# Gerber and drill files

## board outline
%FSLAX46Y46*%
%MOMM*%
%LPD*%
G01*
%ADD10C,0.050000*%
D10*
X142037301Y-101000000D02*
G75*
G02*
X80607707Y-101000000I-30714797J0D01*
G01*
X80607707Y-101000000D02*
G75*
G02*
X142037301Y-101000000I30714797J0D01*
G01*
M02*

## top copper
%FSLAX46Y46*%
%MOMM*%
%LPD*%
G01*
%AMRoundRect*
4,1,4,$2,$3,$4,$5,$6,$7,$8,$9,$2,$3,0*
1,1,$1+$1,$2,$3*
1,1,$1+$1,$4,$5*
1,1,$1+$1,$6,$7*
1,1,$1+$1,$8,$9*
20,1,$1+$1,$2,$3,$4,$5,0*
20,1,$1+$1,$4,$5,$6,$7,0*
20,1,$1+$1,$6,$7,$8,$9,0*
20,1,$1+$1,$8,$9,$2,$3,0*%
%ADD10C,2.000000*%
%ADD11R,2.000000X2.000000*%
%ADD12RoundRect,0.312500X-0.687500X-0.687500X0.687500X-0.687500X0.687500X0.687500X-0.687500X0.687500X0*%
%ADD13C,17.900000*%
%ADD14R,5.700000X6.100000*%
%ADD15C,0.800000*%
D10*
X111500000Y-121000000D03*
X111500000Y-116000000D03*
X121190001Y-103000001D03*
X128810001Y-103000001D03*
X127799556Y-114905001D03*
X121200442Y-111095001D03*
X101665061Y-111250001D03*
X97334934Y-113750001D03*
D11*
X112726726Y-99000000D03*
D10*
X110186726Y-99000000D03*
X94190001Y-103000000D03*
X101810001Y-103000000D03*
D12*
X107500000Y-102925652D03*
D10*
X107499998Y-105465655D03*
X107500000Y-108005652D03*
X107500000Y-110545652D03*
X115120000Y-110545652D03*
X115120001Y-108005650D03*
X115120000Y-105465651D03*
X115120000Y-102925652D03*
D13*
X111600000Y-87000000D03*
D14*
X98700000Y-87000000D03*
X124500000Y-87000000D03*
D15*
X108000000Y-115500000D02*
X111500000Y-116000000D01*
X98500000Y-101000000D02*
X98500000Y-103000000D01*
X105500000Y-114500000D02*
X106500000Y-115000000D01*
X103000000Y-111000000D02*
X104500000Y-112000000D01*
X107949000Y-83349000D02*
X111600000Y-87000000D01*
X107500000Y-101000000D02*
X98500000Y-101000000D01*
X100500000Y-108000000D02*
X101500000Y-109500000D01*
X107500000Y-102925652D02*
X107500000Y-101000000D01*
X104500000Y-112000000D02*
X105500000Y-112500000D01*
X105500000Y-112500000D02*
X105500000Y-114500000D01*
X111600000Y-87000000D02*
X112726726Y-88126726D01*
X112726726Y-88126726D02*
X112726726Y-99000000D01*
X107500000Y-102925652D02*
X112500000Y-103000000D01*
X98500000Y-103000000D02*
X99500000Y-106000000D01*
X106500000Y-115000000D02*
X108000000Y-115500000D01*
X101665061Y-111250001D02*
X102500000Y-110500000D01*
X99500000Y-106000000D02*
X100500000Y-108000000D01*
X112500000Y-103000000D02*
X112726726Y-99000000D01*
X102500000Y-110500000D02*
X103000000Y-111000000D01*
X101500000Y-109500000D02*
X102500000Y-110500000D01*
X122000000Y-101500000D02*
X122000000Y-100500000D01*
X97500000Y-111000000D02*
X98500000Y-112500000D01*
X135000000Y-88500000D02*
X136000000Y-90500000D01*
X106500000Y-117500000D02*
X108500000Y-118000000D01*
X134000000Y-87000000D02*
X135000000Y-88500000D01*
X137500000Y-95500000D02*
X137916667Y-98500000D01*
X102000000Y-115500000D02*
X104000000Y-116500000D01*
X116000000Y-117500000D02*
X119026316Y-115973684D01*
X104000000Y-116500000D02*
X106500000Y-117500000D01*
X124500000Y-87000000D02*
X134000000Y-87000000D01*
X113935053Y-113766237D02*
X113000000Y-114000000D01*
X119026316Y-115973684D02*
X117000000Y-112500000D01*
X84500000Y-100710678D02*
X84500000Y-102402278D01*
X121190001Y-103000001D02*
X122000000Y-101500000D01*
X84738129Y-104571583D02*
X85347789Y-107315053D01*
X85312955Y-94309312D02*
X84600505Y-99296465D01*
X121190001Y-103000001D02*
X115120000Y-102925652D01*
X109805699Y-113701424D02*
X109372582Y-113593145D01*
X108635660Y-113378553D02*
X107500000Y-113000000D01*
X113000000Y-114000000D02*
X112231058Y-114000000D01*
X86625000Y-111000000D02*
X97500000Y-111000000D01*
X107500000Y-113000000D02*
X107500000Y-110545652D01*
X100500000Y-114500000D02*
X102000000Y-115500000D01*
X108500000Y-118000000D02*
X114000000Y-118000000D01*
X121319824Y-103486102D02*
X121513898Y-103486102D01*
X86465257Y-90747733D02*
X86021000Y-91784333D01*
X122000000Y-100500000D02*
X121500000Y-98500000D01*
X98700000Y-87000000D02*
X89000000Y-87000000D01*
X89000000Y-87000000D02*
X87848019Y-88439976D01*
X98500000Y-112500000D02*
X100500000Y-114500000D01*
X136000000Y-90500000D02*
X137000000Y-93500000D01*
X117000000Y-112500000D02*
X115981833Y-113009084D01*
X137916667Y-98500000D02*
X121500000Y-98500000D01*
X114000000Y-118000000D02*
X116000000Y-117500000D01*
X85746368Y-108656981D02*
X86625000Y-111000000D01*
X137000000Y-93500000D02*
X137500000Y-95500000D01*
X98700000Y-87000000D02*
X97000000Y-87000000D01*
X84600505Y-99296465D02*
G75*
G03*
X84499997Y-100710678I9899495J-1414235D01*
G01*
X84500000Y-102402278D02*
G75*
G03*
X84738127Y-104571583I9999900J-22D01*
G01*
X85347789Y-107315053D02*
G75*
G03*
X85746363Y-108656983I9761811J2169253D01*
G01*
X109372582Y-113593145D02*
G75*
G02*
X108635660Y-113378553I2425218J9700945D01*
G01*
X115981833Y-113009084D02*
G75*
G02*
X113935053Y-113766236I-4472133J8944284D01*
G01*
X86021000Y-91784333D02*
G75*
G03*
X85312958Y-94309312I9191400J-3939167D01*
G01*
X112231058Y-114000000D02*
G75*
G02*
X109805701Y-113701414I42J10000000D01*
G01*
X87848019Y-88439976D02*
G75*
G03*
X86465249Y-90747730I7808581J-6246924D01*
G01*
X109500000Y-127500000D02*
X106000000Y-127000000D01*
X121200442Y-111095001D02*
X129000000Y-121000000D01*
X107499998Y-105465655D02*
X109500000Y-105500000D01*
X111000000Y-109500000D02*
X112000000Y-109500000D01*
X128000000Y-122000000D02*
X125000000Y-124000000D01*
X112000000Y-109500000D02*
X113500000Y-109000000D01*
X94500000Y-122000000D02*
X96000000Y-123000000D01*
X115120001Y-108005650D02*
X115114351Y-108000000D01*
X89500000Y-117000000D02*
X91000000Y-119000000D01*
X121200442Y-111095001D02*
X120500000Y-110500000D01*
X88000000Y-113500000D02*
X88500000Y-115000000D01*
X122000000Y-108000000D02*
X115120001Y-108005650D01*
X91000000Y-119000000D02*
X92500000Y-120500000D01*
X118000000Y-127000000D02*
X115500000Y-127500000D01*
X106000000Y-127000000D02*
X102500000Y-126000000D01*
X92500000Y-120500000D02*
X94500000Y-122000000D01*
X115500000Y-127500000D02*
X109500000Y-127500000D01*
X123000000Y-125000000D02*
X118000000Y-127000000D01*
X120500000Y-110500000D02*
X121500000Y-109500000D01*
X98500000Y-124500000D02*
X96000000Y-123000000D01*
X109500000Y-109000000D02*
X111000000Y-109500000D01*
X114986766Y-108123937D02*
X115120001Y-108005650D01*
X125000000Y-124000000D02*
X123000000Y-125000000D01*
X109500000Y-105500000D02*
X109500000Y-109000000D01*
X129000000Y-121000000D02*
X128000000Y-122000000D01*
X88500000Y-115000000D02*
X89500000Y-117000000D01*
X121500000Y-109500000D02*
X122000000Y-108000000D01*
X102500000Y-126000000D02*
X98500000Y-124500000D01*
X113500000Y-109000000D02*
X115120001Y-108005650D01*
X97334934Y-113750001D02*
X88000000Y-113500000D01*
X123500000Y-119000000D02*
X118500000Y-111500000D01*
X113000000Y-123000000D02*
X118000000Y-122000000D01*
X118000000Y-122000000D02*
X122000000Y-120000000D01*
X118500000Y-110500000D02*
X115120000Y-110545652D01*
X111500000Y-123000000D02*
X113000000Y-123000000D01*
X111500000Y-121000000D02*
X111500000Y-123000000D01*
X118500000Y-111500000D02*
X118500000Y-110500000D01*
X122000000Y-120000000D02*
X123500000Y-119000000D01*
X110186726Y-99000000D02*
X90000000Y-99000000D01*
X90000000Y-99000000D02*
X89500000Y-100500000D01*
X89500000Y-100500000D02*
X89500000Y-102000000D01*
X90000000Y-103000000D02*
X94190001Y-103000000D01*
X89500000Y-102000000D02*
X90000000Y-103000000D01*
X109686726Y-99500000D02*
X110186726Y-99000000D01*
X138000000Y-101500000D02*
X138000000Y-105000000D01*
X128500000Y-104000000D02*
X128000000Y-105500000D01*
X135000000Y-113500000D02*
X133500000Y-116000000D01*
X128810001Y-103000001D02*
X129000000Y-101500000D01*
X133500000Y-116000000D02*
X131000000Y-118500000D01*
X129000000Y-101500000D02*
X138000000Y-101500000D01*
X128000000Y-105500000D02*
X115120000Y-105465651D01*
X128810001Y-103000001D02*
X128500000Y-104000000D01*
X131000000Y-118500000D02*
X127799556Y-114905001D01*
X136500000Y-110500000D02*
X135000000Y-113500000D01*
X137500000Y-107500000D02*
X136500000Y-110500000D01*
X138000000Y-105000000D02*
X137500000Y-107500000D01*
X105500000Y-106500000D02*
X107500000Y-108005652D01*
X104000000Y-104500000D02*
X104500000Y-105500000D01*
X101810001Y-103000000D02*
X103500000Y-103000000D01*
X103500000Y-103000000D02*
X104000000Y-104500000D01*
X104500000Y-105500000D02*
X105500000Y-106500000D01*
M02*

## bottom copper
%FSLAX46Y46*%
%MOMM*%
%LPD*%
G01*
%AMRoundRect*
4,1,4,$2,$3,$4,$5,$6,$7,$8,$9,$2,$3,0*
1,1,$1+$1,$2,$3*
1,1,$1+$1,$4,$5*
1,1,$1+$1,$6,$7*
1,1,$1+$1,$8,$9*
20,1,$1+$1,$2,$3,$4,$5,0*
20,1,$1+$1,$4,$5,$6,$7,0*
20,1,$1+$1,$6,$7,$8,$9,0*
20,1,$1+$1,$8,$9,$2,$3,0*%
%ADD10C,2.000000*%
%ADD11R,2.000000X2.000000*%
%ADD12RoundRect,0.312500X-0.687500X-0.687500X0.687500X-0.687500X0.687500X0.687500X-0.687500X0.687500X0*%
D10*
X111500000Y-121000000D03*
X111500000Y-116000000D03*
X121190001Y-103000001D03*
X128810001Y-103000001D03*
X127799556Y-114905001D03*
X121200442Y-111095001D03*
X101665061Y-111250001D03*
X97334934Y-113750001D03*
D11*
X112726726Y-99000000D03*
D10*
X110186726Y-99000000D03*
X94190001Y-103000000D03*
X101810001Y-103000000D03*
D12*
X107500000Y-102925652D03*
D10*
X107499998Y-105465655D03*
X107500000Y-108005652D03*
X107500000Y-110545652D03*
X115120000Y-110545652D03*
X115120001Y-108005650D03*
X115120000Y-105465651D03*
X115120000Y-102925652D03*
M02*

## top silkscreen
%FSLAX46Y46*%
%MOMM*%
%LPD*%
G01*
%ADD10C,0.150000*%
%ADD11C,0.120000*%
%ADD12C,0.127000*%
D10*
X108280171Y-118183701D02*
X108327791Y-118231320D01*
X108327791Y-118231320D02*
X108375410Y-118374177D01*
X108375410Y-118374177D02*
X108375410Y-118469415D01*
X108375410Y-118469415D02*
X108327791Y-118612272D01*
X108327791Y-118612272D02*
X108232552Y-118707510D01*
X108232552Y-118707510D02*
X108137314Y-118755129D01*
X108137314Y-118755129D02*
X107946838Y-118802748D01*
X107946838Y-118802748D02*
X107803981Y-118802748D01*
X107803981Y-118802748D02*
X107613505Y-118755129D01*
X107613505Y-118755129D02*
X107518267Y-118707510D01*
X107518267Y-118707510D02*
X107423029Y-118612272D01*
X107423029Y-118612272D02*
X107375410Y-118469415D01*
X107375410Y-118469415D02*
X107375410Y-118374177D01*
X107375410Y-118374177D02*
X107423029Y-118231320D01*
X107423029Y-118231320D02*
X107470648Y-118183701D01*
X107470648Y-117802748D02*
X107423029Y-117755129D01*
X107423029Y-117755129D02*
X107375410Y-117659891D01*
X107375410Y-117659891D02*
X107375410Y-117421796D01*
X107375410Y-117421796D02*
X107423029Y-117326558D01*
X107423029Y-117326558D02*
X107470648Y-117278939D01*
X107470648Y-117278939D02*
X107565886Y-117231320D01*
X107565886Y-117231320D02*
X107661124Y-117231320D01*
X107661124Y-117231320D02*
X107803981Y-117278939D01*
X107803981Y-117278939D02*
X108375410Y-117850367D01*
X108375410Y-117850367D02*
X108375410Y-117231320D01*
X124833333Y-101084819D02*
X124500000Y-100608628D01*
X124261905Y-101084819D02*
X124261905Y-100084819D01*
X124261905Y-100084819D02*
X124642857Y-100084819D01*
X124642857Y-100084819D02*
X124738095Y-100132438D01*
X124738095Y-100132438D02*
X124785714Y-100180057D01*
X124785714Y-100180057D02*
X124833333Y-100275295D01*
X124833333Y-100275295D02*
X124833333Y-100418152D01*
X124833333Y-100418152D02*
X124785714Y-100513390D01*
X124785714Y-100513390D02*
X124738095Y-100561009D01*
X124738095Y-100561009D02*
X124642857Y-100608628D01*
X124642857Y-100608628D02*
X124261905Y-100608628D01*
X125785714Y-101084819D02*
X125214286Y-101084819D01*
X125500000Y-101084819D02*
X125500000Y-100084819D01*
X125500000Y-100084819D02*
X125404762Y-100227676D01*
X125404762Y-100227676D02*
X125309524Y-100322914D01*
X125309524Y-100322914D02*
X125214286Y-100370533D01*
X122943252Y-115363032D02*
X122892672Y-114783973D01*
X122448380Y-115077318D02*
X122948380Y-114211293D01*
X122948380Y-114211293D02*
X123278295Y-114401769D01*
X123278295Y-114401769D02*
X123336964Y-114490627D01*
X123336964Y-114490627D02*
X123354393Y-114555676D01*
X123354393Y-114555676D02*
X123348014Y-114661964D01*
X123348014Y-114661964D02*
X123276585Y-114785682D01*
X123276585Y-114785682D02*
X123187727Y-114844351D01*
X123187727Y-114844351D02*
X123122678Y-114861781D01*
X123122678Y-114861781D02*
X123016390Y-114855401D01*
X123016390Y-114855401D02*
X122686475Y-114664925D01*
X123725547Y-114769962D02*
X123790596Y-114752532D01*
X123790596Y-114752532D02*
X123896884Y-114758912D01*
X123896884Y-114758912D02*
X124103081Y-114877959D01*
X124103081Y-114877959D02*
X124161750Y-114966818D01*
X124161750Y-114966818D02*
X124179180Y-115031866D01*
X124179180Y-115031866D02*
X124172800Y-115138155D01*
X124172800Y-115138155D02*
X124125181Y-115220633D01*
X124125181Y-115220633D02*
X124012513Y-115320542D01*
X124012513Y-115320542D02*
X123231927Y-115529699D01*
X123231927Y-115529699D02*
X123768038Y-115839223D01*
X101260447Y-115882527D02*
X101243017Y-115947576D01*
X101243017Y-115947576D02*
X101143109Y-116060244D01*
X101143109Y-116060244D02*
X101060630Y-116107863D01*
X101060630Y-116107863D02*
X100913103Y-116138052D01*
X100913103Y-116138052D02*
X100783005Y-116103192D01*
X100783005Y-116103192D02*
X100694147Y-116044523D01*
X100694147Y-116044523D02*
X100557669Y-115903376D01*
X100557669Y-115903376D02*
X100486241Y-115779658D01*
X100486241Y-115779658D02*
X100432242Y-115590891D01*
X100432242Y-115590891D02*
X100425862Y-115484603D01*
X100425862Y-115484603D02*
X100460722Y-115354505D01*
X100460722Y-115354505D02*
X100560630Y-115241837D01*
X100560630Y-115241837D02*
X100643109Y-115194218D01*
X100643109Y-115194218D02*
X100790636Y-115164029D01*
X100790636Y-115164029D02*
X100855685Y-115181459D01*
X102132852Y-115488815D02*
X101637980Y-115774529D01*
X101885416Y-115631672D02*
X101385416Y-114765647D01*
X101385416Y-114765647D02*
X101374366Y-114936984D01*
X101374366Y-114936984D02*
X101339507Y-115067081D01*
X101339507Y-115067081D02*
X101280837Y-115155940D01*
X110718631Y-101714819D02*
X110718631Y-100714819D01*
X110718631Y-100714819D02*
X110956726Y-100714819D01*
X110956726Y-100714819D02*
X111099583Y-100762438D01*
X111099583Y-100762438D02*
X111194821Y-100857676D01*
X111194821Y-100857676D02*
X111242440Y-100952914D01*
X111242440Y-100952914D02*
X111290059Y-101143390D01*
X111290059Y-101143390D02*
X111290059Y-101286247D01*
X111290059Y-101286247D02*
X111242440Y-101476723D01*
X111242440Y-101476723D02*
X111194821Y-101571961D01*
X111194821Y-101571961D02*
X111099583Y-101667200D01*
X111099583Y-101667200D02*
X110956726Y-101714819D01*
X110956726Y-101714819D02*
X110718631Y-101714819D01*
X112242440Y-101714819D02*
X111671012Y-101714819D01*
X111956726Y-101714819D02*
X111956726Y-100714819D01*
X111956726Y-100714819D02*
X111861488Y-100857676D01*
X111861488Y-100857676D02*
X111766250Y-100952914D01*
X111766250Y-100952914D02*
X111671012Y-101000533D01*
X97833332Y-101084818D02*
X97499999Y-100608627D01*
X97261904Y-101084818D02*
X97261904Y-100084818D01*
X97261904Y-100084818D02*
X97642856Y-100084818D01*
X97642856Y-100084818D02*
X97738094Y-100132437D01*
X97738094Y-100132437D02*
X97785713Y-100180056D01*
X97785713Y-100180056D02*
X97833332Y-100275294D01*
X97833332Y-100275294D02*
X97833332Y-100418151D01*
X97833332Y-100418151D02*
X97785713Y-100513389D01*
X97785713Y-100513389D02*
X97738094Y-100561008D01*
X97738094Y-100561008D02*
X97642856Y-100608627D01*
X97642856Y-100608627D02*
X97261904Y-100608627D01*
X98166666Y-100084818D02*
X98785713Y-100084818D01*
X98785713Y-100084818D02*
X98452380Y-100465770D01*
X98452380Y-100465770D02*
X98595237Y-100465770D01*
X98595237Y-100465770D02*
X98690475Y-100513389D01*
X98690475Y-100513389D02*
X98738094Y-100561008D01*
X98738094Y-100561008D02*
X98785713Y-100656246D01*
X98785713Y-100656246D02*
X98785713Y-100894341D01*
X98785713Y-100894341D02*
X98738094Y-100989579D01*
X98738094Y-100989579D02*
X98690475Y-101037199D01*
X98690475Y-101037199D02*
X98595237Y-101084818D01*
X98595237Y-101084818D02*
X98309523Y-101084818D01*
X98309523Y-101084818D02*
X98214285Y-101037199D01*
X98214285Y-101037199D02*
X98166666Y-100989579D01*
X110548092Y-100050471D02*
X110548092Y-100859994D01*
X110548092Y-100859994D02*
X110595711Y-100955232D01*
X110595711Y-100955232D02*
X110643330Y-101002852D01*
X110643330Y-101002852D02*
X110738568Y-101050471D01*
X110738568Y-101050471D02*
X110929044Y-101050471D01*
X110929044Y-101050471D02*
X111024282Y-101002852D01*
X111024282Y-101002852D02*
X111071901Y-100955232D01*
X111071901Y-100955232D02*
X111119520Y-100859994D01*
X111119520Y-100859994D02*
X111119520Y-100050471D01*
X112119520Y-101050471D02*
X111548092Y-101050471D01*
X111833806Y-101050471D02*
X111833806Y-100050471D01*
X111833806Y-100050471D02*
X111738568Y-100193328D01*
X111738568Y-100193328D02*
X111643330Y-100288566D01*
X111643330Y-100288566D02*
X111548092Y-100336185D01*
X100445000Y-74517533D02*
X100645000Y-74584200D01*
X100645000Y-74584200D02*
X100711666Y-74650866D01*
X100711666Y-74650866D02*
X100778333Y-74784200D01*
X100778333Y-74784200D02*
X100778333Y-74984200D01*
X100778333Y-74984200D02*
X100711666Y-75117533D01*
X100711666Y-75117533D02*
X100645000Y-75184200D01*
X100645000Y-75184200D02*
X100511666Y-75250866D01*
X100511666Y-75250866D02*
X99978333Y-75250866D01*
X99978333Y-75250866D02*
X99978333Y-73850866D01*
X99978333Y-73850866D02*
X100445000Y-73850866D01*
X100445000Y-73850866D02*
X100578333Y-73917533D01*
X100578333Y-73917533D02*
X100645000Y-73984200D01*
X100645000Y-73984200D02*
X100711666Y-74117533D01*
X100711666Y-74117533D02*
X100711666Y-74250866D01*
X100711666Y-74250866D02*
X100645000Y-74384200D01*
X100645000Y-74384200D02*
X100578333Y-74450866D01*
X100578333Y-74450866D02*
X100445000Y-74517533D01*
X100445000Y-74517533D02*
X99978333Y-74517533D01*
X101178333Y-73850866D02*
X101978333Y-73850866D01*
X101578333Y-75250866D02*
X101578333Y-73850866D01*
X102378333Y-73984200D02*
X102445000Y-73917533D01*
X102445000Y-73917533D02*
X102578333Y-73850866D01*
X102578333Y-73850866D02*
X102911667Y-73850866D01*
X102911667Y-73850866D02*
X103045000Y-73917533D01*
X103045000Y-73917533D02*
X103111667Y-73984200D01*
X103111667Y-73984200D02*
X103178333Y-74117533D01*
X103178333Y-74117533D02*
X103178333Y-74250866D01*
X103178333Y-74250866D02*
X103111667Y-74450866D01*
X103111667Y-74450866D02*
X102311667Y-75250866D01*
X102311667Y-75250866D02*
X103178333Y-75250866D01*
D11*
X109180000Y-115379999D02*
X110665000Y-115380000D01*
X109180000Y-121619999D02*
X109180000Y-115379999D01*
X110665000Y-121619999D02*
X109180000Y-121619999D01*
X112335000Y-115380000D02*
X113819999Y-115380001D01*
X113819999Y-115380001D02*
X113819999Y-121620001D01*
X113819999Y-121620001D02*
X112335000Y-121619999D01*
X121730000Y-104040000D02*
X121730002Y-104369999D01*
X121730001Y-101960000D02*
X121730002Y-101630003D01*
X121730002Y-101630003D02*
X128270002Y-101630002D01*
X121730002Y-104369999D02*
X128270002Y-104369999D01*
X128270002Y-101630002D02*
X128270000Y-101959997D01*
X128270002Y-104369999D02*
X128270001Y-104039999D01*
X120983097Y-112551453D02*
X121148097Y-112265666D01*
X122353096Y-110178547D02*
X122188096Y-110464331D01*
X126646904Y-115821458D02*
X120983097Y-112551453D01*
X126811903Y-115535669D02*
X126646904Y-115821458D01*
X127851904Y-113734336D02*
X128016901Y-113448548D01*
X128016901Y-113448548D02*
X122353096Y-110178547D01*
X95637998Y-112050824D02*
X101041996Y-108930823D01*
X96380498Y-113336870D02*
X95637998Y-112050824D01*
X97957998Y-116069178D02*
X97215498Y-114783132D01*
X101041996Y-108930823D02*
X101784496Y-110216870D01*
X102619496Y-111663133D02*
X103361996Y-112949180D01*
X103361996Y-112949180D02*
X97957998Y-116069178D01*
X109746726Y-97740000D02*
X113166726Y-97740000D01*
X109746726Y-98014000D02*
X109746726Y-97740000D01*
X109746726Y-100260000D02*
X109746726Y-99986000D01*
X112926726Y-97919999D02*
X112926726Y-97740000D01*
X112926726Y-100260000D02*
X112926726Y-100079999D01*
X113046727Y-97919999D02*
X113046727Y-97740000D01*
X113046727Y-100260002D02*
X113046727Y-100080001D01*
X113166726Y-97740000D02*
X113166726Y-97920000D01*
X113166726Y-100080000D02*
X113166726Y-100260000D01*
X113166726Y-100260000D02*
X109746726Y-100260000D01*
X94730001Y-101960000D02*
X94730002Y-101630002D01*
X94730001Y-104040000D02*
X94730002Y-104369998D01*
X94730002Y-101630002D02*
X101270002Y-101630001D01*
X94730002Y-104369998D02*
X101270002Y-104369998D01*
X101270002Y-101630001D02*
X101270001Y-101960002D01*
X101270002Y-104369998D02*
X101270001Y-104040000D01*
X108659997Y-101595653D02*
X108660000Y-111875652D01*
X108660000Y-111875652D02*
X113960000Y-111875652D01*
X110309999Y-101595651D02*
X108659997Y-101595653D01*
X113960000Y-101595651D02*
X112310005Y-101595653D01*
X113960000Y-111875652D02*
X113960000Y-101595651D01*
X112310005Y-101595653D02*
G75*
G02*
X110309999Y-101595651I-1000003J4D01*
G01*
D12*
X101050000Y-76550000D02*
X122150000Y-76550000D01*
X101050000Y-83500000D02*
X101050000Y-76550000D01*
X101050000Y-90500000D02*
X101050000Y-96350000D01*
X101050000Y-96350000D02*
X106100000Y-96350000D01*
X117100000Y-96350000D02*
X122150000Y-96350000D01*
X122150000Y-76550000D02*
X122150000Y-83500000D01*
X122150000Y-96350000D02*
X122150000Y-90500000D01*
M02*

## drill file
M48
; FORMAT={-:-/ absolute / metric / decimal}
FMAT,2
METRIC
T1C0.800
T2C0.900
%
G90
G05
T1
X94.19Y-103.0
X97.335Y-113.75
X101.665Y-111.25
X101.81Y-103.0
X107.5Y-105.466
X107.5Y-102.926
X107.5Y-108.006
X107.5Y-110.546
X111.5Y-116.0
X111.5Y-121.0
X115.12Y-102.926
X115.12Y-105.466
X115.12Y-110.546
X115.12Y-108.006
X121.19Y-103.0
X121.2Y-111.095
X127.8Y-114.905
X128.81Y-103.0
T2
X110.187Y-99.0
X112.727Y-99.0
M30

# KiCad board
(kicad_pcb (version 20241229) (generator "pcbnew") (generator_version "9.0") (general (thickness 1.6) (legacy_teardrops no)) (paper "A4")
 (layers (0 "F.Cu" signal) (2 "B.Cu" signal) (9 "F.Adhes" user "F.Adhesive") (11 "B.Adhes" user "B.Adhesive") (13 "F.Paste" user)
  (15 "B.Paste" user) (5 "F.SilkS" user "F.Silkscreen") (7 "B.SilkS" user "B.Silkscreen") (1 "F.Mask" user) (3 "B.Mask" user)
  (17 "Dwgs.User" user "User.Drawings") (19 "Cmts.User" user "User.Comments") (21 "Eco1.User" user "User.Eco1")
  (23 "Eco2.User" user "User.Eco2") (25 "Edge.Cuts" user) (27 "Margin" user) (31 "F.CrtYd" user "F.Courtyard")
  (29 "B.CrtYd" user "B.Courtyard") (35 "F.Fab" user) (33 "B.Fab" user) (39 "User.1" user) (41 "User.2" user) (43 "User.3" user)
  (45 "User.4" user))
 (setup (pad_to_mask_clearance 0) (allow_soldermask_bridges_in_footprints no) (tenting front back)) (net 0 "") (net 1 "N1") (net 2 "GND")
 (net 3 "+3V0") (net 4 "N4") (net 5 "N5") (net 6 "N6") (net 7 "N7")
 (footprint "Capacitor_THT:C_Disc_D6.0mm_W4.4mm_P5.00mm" (layer "F.Cu") (at 111.5 121 90)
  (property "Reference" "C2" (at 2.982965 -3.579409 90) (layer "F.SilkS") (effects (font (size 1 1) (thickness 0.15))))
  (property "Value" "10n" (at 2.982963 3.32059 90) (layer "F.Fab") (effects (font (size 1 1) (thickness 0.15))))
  (fp_line (start 5.620001 -2.32) (end 5.62 -0.835) (stroke (width 0.12) (type solid)) (layer "F.SilkS"))
  (fp_line (start -0.619999 -2.32) (end 5.620001 -2.32) (stroke (width 0.12) (type solid)) (layer "F.SilkS"))
  (fp_line (start -0.619999 -0.835) (end -0.619999 -2.32) (stroke (width 0.12) (type solid)) (layer "F.SilkS"))
  (fp_line (start 5.62 0.835) (end 5.619999 2.319999) (stroke (width 0.12) (type solid)) (layer "F.SilkS"))
  (fp_line (start 5.619999 2.319999) (end -0.620001 2.319999) (stroke (width 0.12) (type solid)) (layer "F.SilkS"))
  (fp_line (start -0.620001 2.319999) (end -0.619999 0.835) (stroke (width 0.12) (type solid)) (layer "F.SilkS"))
  (pad "1" thru_hole circle (at 0 0 90) (size 2 2) (drill 0.8) (layers "*.Cu" "*.Mask") (remove_unused_layers no) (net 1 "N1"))
  (pad "2" thru_hole circle (at 5 0 90) (size 2 2) (drill 0.8) (layers "*.Cu" "*.Mask") (remove_unused_layers no) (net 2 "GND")))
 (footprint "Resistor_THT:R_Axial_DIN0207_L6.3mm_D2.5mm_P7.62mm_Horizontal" (layer "F.Cu") (at 121.190001 103.000001)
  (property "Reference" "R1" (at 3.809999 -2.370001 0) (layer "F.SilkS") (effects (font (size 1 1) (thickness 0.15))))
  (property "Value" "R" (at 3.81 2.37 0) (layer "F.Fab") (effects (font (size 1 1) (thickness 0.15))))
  (fp_line (start 0.539999 1.039999) (end 0.540001 1.369998) (stroke (width 0.12) (type solid)) (layer "F.SilkS"))
  (fp_line (start 0.54 -1.040001) (end 0.540001 -1.369998) (stroke (width 0.12) (type solid)) (layer "F.SilkS"))
  (fp_line (start 0.540001 -1.369998) (end 7.080001 -1.369999) (stroke (width 0.12) (type solid)) (layer "F.SilkS"))
  (fp_line (start 0.540001 1.369998) (end 7.080001 1.369998) (stroke (width 0.12) (type solid)) (layer "F.SilkS"))
  (fp_line (start 7.080001 -1.369999) (end 7.079999 -1.040004) (stroke (width 0.12) (type solid)) (layer "F.SilkS"))
  (fp_line (start 7.080001 1.369998) (end 7.08 1.039998) (stroke (width 0.12) (type solid)) (layer "F.SilkS"))
  (pad "1" thru_hole circle (at 0 0) (size 2 2) (drill 0.8) (layers "*.Cu" "*.Mask") (remove_unused_layers no) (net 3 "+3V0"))
  (pad "2" thru_hole circle (at 7.62 0) (size 2 2) (drill 0.8) (layers "*.Cu" "*.Mask") (remove_unused_layers no) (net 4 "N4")))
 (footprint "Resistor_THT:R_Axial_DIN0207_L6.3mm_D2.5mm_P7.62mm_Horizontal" (layer "F.Cu") (at 127.799556 114.905001 150)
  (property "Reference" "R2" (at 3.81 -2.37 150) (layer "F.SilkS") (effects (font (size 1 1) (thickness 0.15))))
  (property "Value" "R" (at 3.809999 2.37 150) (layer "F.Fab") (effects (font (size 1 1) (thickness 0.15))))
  (fp_line (start 7.080001 -1.369997) (end 7.08 -1.039998) (stroke (width 0.12) (type solid)) (layer "F.SilkS"))
  (fp_line (start 7.08 1.369999) (end 7.080002 1.040003) (stroke (width 0.12) (type solid)) (layer "F.SilkS"))
  (fp_line (start 0.539997 -1.370001) (end 7.080001 -1.369997) (stroke (width 0.12) (type solid)) (layer "F.SilkS"))
  (fp_line (start 0.539999 -1.040001) (end 0.539997 -1.370001) (stroke (width 0.12) (type solid)) (layer "F.SilkS"))
  (fp_line (start 0.539998 1.04) (end 0.54 1.369998) (stroke (width 0.12) (type solid)) (layer "F.SilkS"))
  (fp_line (start 0.54 1.369998) (end 7.08 1.369999) (stroke (width 0.12) (type solid)) (layer "F.SilkS"))
  (pad "1" thru_hole circle (at 0 0 150) (size 2 2) (drill 0.8) (layers "*.Cu" "*.Mask") (remove_unused_layers no) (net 4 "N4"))
  (pad "2" thru_hole circle (at 7.62 0 150) (size 2 2) (drill 0.8) (layers "*.Cu" "*.Mask") (remove_unused_layers no) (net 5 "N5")))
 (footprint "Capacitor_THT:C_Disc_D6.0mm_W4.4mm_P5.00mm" (layer "F.Cu") (at 101.665061 111.250001 -150)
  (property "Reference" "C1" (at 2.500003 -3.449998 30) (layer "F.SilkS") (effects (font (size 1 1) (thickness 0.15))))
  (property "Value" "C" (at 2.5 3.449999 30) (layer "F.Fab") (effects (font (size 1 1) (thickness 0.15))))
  (fp_line (start 5.620001 2.319998) (end -0.619999 2.32) (stroke (width 0.12) (type solid)) (layer "F.SilkS"))
  (fp_line (start 5.62 0.835) (end 5.620001 2.319998) (stroke (width 0.12) (type solid)) (layer "F.SilkS"))
  (fp_line (start 5.619999 -2.319998) (end 5.62 -0.835) (stroke (width 0.12) (type solid)) (layer "F.SilkS"))
  (fp_line (start -0.619999 2.32) (end -0.619999 0.835) (stroke (width 0.12) (type solid)) (layer "F.SilkS"))
  (fp_line (start -0.619999 -0.835) (end -0.619999 -2.32) (stroke (width 0.12) (type solid)) (layer "F.SilkS"))
  (fp_line (start -0.619999 -2.32) (end 5.619999 -2.319998) (stroke (width 0.12) (type solid)) (layer "F.SilkS"))
  (pad "1" thru_hole circle (at 0 0 210) (size 2 2) (drill 0.8) (layers "*.Cu" "*.Mask") (remove_unused_layers no) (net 2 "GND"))
  (pad "2" thru_hole circle (at 5 0 210) (size 2 2) (drill 0.8) (layers "*.Cu" "*.Mask") (remove_unused_layers no) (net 5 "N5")))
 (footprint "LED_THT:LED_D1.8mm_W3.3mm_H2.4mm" (layer "F.Cu") (at 112.726726 99 180)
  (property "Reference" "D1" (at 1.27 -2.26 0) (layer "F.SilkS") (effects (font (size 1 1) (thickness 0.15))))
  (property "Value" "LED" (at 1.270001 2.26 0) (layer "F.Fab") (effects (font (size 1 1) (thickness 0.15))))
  (fp_line (start 2.98 1.26) (end -0.44 1.26) (stroke (width 0.12) (type solid)) (layer "F.SilkS"))
  (fp_line (start 2.98 0.986) (end 2.98 1.26) (stroke (width 0.12) (type solid)) (layer "F.SilkS"))
  (fp_line (start 2.98 -1.26) (end 2.98 -0.986) (stroke (width 0.12) (type solid)) (layer "F.SilkS"))
  (fp_line (start -0.2 1.080001) (end -0.2 1.26) (stroke (width 0.12) (type solid)) (layer "F.SilkS"))
  (fp_line (start -0.2 -1.26) (end -0.2 -1.079999) (stroke (width 0.12) (type solid)) (layer "F.SilkS"))
  (fp_line (start -0.320001 1.080001) (end -0.320001 1.26) (stroke (width 0.12) (type solid)) (layer "F.SilkS"))
  (fp_line (start -0.320001 -1.260002) (end -0.320001 -1.080001) (stroke (width 0.12) (type solid)) (layer "F.SilkS"))
  (fp_line (start -0.44 1.26) (end -0.44 1.08) (stroke (width 0.12) (type solid)) (layer "F.SilkS"))
  (fp_line (start -0.44 -1.08) (end -0.44 -1.26) (stroke (width 0.12) (type solid)) (layer "F.SilkS"))
  (fp_line (start -0.44 -1.26) (end 2.98 -1.26) (stroke (width 0.12) (type solid)) (layer "F.SilkS"))
  (pad "1" thru_hole rect (at 0 0 180) (size 2 2) (drill 0.9) (layers "*.Cu" "*.Mask") (remove_unused_layers no) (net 2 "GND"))
  (pad "2" thru_hole circle (at 2.54 0 180) (size 2 2) (drill 0.9) (layers "*.Cu" "*.Mask") (remove_unused_layers no) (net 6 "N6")))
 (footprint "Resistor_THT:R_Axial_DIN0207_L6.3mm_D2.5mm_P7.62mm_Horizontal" (layer "F.Cu") (at 94.190001 103)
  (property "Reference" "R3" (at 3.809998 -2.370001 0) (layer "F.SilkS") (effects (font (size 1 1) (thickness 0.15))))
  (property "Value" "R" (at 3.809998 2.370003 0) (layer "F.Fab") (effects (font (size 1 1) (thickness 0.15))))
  (fp_line (start 0.54 -1.04) (end 0.540001 -1.369998) (stroke (width 0.12) (type solid)) (layer "F.SilkS"))
  (fp_line (start 0.54 1.04) (end 0.540001 1.369998) (stroke (width 0.12) (type solid)) (layer "F.SilkS"))
  (fp_line (start 0.540001 -1.369998) (end 7.080001 -1.369999) (stroke (width 0.12) (type solid)) (layer "F.SilkS"))
  (fp_line (start 0.540001 1.369998) (end 7.080001 1.369998) (stroke (width 0.12) (type solid)) (layer "F.SilkS"))
  (fp_line (start 7.080001 -1.369999) (end 7.08 -1.039998) (stroke (width 0.12) (type solid)) (layer "F.SilkS"))
  (fp_line (start 7.080001 1.369998) (end 7.08 1.04) (stroke (width 0.12) (type solid)) (layer "F.SilkS"))
  (pad "1" thru_hole circle (at 0 0) (size 2 2) (drill 0.8) (layers "*.Cu" "*.Mask") (remove_unused_layers no) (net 6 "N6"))
  (pad "2" thru_hole circle (at 7.62 0) (size 2 2) (drill 0.8) (layers "*.Cu" "*.Mask") (remove_unused_layers no) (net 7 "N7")))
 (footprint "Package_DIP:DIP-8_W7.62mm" (layer "F.Cu") (at 107.5 102.925652)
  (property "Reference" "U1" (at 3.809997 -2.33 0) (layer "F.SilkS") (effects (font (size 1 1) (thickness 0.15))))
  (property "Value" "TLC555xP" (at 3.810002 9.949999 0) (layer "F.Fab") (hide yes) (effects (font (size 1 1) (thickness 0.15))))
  (fp_line (start 1.159997 -1.329999) (end 1.16 8.95) (stroke (width 0.12) (type solid)) (layer "F.SilkS"))
  (fp_line (start 1.16 8.95) (end 6.46 8.95) (stroke (width 0.12) (type solid)) (layer "F.SilkS"))
  (fp_line (start 2.809999 -1.330001) (end 1.159997 -1.329999) (stroke (width 0.12) (type solid)) (layer "F.SilkS"))
  (fp_line (start 6.46 -1.330001) (end 4.810005 -1.329999) (stroke (width 0.12) (type solid)) (layer "F.SilkS"))
  (fp_line (start 6.46 8.95) (end 6.46 -1.330001) (stroke (width 0.12) (type solid)) (layer "F.SilkS"))
  (fp_arc (start 4.810005 -1.329999) (mid 3.81 -0.33) (end 2.809999 -1.330001) (stroke (width 0.12) (type solid)) (layer "F.SilkS"))
  (pad "1" thru_hole roundrect (at 0 0) (size 2 2) (drill 0.8) (layers "*.Cu" "*.Mask") (remove_unused_layers no) (roundrect_rratio 0.15625)
   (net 2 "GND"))
  (pad "2" thru_hole circle (at -0.000002 2.540003) (size 2 2) (drill 0.8) (layers "*.Cu" "*.Mask") (remove_unused_layers no) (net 5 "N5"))
  (pad "3" thru_hole circle (at 0 5.08) (size 2 2) (drill 0.8) (layers "*.Cu" "*.Mask") (remove_unused_layers no) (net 7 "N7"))
  (pad "4" thru_hole circle (at 0 7.62) (size 2 2) (drill 0.8) (layers "*.Cu" "*.Mask") (remove_unused_layers no) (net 3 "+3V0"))
  (pad "5" thru_hole circle (at 7.62 7.62) (size 2 2) (drill 0.8) (layers "*.Cu" "*.Mask") (remove_unused_layers no) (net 1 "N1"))
  (pad "6" thru_hole circle (at 7.620001 5.079998) (size 2 2) (drill 0.8) (layers "*.Cu" "*.Mask") (remove_unused_layers no) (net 5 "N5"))
  (pad "7" thru_hole circle (at 7.62 2.539999) (size 2 2) (drill 0.8) (layers "*.Cu" "*.Mask") (remove_unused_layers no) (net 4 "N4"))
  (pad "8" thru_hole circle (at 7.62 0) (size 2 2) (drill 0.8) (layers "*.Cu" "*.Mask") (remove_unused_layers no) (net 3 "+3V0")))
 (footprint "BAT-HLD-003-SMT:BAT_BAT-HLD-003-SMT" (layer "F.Cu") (at 111.6 87)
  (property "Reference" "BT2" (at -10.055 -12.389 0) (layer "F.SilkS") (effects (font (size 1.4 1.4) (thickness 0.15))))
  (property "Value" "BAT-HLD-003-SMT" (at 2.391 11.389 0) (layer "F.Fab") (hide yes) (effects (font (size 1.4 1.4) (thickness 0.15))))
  (fp_line (start -10.55 -10.45) (end 10.55 -10.45) (stroke (width 0.127) (type solid)) (layer "F.SilkS"))
  (fp_line (start -10.55 -3.5) (end -10.55 -10.45) (stroke (width 0.127) (type solid)) (layer "F.SilkS"))
  (fp_line (start -10.55 3.5) (end -10.55 9.35) (stroke (width 0.127) (type solid)) (layer "F.SilkS"))
  (fp_line (start -10.55 9.35) (end -5.5 9.35) (stroke (width 0.127) (type solid)) (layer "F.SilkS"))
  (fp_line (start 5.5 9.35) (end 10.55 9.35) (stroke (width 0.127) (type solid)) (layer "F.SilkS"))
  (fp_line (start 10.55 -10.45) (end 10.55 -3.5) (stroke (width 0.127) (type solid)) (layer "F.SilkS"))
  (fp_line (start 10.55 9.35) (end 10.55 3.5) (stroke (width 0.127) (type solid)) (layer "F.SilkS"))
  (pad "N" smd circle (at 0 0) (size 17.9 17.9) (layers "F.Cu" "F.Mask") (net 2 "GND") (solder_mask_margin 0.102))
  (pad "P1" smd rect (at -12.9 0) (size 5.7 6.1) (layers "F.Cu" "F.Mask" "F.Paste") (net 3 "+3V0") (solder_mask_margin 0.102))
  (pad "P2" smd rect (at 12.9 0) (size 5.7 6.1) (layers "F.Cu" "F.Mask" "F.Paste") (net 3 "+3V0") (solder_mask_margin 0.102)))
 (gr_circle (center 111.322504 101) (end 140 112) (stroke (width 0.05) (type default)) (fill no) (layer "Edge.Cuts"))
 (segment (start 108 115.5) (end 111.5 116) (width 0.8) (layer "F.Cu") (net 2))
 (segment (start 98.5 101) (end 98.5 103) (width 0.8) (layer "F.Cu") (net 2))
 (segment (start 105.5 114.5) (end 106.5 115) (width 0.8) (layer "F.Cu") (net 2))
 (segment (start 103 111) (end 104.5 112) (width 0.8) (layer "F.Cu") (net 2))
 (segment (start 107.949 83.349) (end 111.6 87) (width 0.8) (layer "F.Cu") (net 2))
 (segment (start 107.5 101) (end 98.5 101) (width 0.8) (layer "F.Cu") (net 2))
 (segment (start 100.5 108) (end 101.5 109.5) (width 0.8) (layer "F.Cu") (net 2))
 (segment (start 107.5 102.925652) (end 107.5 101) (width 0.8) (layer "F.Cu") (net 2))
 (segment (start 104.5 112) (end 105.5 112.5) (width 0.8) (layer "F.Cu") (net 2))
 (segment (start 105.5 112.5) (end 105.5 114.5) (width 0.8) (layer "F.Cu") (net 2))
 (segment (start 111.6 87) (end 112.726726 88.126726) (width 0.8) (layer "F.Cu") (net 2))
 (segment (start 112.726726 88.126726) (end 112.726726 99) (width 0.8) (layer "F.Cu") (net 2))
 (segment (start 107.5 102.925652) (end 112.5 103) (width 0.8) (layer "F.Cu") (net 2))
 (segment (start 98.5 103) (end 99.5 106) (width 0.8) (layer "F.Cu") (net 2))
 (segment (start 106.5 115) (end 108 115.5) (width 0.8) (layer "F.Cu") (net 2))
 (segment (start 101.665061 111.250001) (end 102.5 110.5) (width 0.8) (layer "F.Cu") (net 2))
 (segment (start 99.5 106) (end 100.5 108) (width 0.8) (layer "F.Cu") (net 2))
 (segment (start 112.5 103) (end 112.726726 99) (width 0.8) (layer "F.Cu") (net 2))
 (segment (start 102.5 110.5) (end 103 111) (width 0.8) (layer "F.Cu") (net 2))
 (segment (start 101.5 109.5) (end 102.5 110.5) (width 0.8) (layer "F.Cu") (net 2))
 (segment (start 122 101.5) (end 122 100.5) (width 0.8) (layer "F.Cu") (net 3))
 (segment (start 97.5 111) (end 98.5 112.5) (width 0.8) (layer "F.Cu") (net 3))
 (segment (start 135 88.5) (end 136 90.5) (width 0.8) (layer "F.Cu") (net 3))
 (segment (start 106.5 117.5) (end 108.5 118) (width 0.8) (layer "F.Cu") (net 3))
 (segment (start 134 87) (end 135 88.5) (width 0.8) (layer "F.Cu") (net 3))
 (segment (start 137.5 95.5) (end 137.916667 98.5) (width 0.8) (layer "F.Cu") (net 3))
 (segment (start 102 115.5) (end 104 116.5) (width 0.8) (layer "F.Cu") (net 3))
 (segment (start 116 117.5) (end 119.026316 115.973684) (width 0.8) (layer "F.Cu") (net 3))
 (segment (start 104 116.5) (end 106.5 117.5) (width 0.8) (layer "F.Cu") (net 3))
 (segment (start 124.5 87) (end 134 87) (width 0.8) (layer "F.Cu") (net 3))
 (segment (start 113.935053 113.766237) (end 113 114) (width 0.8) (layer "F.Cu") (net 3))
 (segment (start 119.026316 115.973684) (end 117 112.5) (width 0.8) (layer "F.Cu") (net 3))
 (segment (start 84.5 100.710678) (end 84.5 102.402278) (width 0.8) (layer "F.Cu") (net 3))
 (segment (start 121.190001 103.000001) (end 122 101.5) (width 0.8) (layer "F.Cu") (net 3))
 (segment (start 84.738129 104.571583) (end 85.347789 107.315053) (width 0.8) (layer "F.Cu") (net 3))
 (segment (start 85.312955 94.309312) (end 84.600505 99.296465) (width 0.8) (layer "F.Cu") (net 3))
 (segment (start 121.190001 103.000001) (end 115.12 102.925652) (width 0.8) (layer "F.Cu") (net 3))
 (segment (start 109.805699 113.701424) (end 109.372582 113.593145) (width 0.8) (layer "F.Cu") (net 3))
 (segment (start 108.63566 113.378553) (end 107.5 113) (width 0.8) (layer "F.Cu") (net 3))
 (segment (start 113 114) (end 112.231058 114) (width 0.8) (layer "F.Cu") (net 3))
 (segment (start 86.625 111) (end 97.5 111) (width 0.8) (layer "F.Cu") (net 3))
 (segment (start 107.5 113) (end 107.5 110.545652) (width 0.8) (layer "F.Cu") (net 3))
 (segment (start 100.5 114.5) (end 102 115.5) (width 0.8) (layer "F.Cu") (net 3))
 (segment (start 108.5 118) (end 114 118) (width 0.8) (layer "F.Cu") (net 3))
 (segment (start 121.319824 103.486102) (end 121.513898 103.486102) (width 0.8) (layer "F.Cu") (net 3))
 (segment (start 86.465257 90.747733) (end 86.021 91.784333) (width 0.8) (layer "F.Cu") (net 3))
 (segment (start 122 100.5) (end 121.5 98.5) (width 0.8) (layer "F.Cu") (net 3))
 (segment (start 98.7 87) (end 89 87) (width 0.8) (layer "F.Cu") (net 3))
 (segment (start 89 87) (end 87.848019 88.439976) (width 0.8) (layer "F.Cu") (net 3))
 (segment (start 98.5 112.5) (end 100.5 114.5) (width 0.8) (layer "F.Cu") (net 3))
 (segment (start 136 90.5) (end 137 93.5) (width 0.8) (layer "F.Cu") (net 3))
 (segment (start 117 112.5) (end 115.981833 113.009084) (width 0.8) (layer "F.Cu") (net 3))
 (segment (start 137.916667 98.5) (end 121.5 98.5) (width 0.8) (layer "F.Cu") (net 3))
 (segment (start 114 118) (end 116 117.5) (width 0.8) (layer "F.Cu") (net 3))
 (segment (start 85.746368 108.656981) (end 86.625 111) (width 0.8) (layer "F.Cu") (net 3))
 (segment (start 137 93.5) (end 137.5 95.5) (width 0.8) (layer "F.Cu") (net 3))
 (segment (start 98.7 87) (end 97 87) (width 0.8) (layer "F.Cu") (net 3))
 (arc (start 84.600505 99.296465) (mid 84.525158 100.001788) (end 84.5 100.710678) (width 0.8) (layer "F.Cu") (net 3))
 (arc (start 84.5 102.402278) (mid 84.55971 103.493446) (end 84.738129 104.571583) (width 0.8) (layer "F.Cu") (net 3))
 (arc (start 85.347789 107.315053) (mid 85.523568 107.993) (end 85.746368 108.656981) (width 0.8) (layer "F.Cu") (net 3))
 (arc (start 109.372582 113.593145) (mid 109.002061 113.492922) (end 108.63566 113.378553) (width 0.8) (layer "F.Cu") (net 3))
 (arc (start 115.981833 113.009084) (mid 114.979159 113.443662) (end 113.935053 113.766237) (width 0.8) (layer "F.Cu") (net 3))
 (arc (start 86.021 91.784333) (mid 85.58385 93.023512) (end 85.312955 94.309312) (width 0.8) (layer "F.Cu") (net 3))
 (arc (start 112.231058 114) (mid 111.009224 113.925075) (end 109.805699 113.701424) (width 0.8) (layer "F.Cu") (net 3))
 (arc (start 87.848019 88.439976) (mid 87.078676 89.547141) (end 86.465257 90.747733) (width 0.8) (layer "F.Cu") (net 3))
 (segment (start 109.5 127.5) (end 106 127) (width 0.8) (layer "F.Cu") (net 5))
 (segment (start 121.200442 111.095001) (end 129 121) (width 0.8) (layer "F.Cu") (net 5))
 (segment (start 107.499998 105.465655) (end 109.5 105.5) (width 0.8) (layer "F.Cu") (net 5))
 (segment (start 111 109.5) (end 112 109.5) (width 0.8) (layer "F.Cu") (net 5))
 (segment (start 128 122) (end 125 124) (width 0.8) (layer "F.Cu") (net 5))
 (segment (start 112 109.5) (end 113.5 109) (width 0.8) (layer "F.Cu") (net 5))
 (segment (start 94.5 122) (end 96 123) (width 0.8) (layer "F.Cu") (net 5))
 (segment (start 115.120001 108.00565) (end 115.114351 108) (width 0.8) (layer "F.Cu") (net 5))
 (segment (start 89.5 117) (end 91 119) (width 0.8) (layer "F.Cu") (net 5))
 (segment (start 121.200442 111.095001) (end 120.5 110.5) (width 0.8) (layer "F.Cu") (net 5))
 (segment (start 88 113.5) (end 88.5 115) (width 0.8) (layer "F.Cu") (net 5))
 (segment (start 122 108) (end 115.120001 108.00565) (width 0.8) (layer "F.Cu") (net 5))
 (segment (start 91 119) (end 92.5 120.5) (width 0.8) (layer "F.Cu") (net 5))
 (segment (start 118 127) (end 115.5 127.5) (width 0.8) (layer "F.Cu") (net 5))
 (segment (start 106 127) (end 102.5 126) (width 0.8) (layer "F.Cu") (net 5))
 (segment (start 92.5 120.5) (end 94.5 122) (width 0.8) (layer "F.Cu") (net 5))
 (segment (start 115.5 127.5) (end 109.5 127.5) (width 0.8) (layer "F.Cu") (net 5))
 (segment (start 123 125) (end 118 127) (width 0.8) (layer "F.Cu") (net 5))
 (segment (start 120.5 110.5) (end 121.5 109.5) (width 0.8) (layer "F.Cu") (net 5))
 (segment (start 98.5 124.5) (end 96 123) (width 0.8) (layer "F.Cu") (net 5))
 (segment (start 109.5 109) (end 111 109.5) (width 0.8) (layer "F.Cu") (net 5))
 (segment (start 114.986766 108.123937) (end 115.120001 108.00565) (width 0.8) (layer "F.Cu") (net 5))
 (segment (start 125 124) (end 123 125) (width 0.8) (layer "F.Cu") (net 5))
 (segment (start 109.5 105.5) (end 109.5 109) (width 0.8) (layer "F.Cu") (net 5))
 (segment (start 129 121) (end 128 122) (width 0.8) (layer "F.Cu") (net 5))
 (segment (start 88.5 115) (end 89.5 117) (width 0.8) (layer "F.Cu") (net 5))
 (segment (start 121.5 109.5) (end 122 108) (width 0.8) (layer "F.Cu") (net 5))
 (segment (start 102.5 126) (end 98.5 124.5) (width 0.8) (layer "F.Cu") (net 5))
 (segment (start 113.5 109) (end 115.120001 108.00565) (width 0.8) (layer "F.Cu") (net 5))
 (segment (start 97.334934 113.750001) (end 88 113.5) (width 0.8) (layer "F.Cu") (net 5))
 (segment (start 123.5 119) (end 118.5 111.5) (width 0.8) (layer "F.Cu") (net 1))
 (segment (start 113 123) (end 118 122) (width 0.8) (layer "F.Cu") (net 1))
 (segment (start 118 122) (end 122 120) (width 0.8) (layer "F.Cu") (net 1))
 (segment (start 118.5 110.5) (end 115.12 110.545652) (width 0.8) (layer "F.Cu") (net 1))
 (segment (start 111.5 123) (end 113 123) (width 0.8) (layer "F.Cu") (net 1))
 (segment (start 111.5 121) (end 111.5 123) (width 0.8) (layer "F.Cu") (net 1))
 (segment (start 118.5 111.5) (end 118.5 110.5) (width 0.8) (layer "F.Cu") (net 1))
 (segment (start 122 120) (end 123.5 119) (width 0.8) (layer "F.Cu") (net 1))
 (segment (start 110.186726 99) (end 90 99) (width 0.8) (layer "F.Cu") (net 6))
 (segment (start 90 99) (end 89.5 100.5) (width 0.8) (layer "F.Cu") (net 6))
 (segment (start 89.5 100.5) (end 89.5 102) (width 0.8) (layer "F.Cu") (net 6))
 (segment (start 90 103) (end 94.190001 103) (width 0.8) (layer "F.Cu") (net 6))
 (segment (start 89.5 102) (end 90 103) (width 0.8) (layer "F.Cu") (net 6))
 (segment (start 109.686726 99.5) (end 110.186726 99) (width 0.8) (layer "F.Cu") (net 6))
 (segment (start 138 101.5) (end 138 105) (width 0.8) (layer "F.Cu") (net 4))
 (segment (start 128.5 104) (end 128 105.5) (width 0.8) (layer "F.Cu") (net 4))
 (segment (start 135 113.5) (end 133.5 116) (width 0.8) (layer "F.Cu") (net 4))
 (segment (start 128.810001 103.000001) (end 129 101.5) (width 0.8) (layer "F.Cu") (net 4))
 (segment (start 133.5 116) (end 131 118.5) (width 0.8) (layer "F.Cu") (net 4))
 (segment (start 129 101.5) (end 138 101.5) (width 0.8) (layer "F.Cu") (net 4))
 (segment (start 128 105.5) (end 115.12 105.465651) (width 0.8) (layer "F.Cu") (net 4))
 (segment (start 128.810001 103.000001) (end 128.5 104) (width 0.8) (layer "F.Cu") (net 4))
 (segment (start 131 118.5) (end 127.799556 114.905001) (width 0.8) (layer "F.Cu") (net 4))
 (segment (start 136.5 110.5) (end 135 113.5) (width 0.8) (layer "F.Cu") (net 4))
 (segment (start 137.5 107.5) (end 136.5 110.5) (width 0.8) (layer "F.Cu") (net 4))
 (segment (start 138 105) (end 137.5 107.5) (width 0.8) (layer "F.Cu") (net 4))
 (segment (start 105.5 106.5) (end 107.5 108.005652) (width 0.8) (layer "F.Cu") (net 7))
 (segment (start 104 104.5) (end 104.5 105.5) (width 0.8) (layer "F.Cu") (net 7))
 (segment (start 101.810001 103) (end 103.5 103) (width 0.8) (layer "F.Cu") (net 7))
 (segment (start 103.5 103) (end 104 104.5) (width 0.8) (layer "F.Cu") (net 7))
 (segment (start 104.5 105.5) (end 105.5 106.5) (width 0.8) (layer "F.Cu") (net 7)))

